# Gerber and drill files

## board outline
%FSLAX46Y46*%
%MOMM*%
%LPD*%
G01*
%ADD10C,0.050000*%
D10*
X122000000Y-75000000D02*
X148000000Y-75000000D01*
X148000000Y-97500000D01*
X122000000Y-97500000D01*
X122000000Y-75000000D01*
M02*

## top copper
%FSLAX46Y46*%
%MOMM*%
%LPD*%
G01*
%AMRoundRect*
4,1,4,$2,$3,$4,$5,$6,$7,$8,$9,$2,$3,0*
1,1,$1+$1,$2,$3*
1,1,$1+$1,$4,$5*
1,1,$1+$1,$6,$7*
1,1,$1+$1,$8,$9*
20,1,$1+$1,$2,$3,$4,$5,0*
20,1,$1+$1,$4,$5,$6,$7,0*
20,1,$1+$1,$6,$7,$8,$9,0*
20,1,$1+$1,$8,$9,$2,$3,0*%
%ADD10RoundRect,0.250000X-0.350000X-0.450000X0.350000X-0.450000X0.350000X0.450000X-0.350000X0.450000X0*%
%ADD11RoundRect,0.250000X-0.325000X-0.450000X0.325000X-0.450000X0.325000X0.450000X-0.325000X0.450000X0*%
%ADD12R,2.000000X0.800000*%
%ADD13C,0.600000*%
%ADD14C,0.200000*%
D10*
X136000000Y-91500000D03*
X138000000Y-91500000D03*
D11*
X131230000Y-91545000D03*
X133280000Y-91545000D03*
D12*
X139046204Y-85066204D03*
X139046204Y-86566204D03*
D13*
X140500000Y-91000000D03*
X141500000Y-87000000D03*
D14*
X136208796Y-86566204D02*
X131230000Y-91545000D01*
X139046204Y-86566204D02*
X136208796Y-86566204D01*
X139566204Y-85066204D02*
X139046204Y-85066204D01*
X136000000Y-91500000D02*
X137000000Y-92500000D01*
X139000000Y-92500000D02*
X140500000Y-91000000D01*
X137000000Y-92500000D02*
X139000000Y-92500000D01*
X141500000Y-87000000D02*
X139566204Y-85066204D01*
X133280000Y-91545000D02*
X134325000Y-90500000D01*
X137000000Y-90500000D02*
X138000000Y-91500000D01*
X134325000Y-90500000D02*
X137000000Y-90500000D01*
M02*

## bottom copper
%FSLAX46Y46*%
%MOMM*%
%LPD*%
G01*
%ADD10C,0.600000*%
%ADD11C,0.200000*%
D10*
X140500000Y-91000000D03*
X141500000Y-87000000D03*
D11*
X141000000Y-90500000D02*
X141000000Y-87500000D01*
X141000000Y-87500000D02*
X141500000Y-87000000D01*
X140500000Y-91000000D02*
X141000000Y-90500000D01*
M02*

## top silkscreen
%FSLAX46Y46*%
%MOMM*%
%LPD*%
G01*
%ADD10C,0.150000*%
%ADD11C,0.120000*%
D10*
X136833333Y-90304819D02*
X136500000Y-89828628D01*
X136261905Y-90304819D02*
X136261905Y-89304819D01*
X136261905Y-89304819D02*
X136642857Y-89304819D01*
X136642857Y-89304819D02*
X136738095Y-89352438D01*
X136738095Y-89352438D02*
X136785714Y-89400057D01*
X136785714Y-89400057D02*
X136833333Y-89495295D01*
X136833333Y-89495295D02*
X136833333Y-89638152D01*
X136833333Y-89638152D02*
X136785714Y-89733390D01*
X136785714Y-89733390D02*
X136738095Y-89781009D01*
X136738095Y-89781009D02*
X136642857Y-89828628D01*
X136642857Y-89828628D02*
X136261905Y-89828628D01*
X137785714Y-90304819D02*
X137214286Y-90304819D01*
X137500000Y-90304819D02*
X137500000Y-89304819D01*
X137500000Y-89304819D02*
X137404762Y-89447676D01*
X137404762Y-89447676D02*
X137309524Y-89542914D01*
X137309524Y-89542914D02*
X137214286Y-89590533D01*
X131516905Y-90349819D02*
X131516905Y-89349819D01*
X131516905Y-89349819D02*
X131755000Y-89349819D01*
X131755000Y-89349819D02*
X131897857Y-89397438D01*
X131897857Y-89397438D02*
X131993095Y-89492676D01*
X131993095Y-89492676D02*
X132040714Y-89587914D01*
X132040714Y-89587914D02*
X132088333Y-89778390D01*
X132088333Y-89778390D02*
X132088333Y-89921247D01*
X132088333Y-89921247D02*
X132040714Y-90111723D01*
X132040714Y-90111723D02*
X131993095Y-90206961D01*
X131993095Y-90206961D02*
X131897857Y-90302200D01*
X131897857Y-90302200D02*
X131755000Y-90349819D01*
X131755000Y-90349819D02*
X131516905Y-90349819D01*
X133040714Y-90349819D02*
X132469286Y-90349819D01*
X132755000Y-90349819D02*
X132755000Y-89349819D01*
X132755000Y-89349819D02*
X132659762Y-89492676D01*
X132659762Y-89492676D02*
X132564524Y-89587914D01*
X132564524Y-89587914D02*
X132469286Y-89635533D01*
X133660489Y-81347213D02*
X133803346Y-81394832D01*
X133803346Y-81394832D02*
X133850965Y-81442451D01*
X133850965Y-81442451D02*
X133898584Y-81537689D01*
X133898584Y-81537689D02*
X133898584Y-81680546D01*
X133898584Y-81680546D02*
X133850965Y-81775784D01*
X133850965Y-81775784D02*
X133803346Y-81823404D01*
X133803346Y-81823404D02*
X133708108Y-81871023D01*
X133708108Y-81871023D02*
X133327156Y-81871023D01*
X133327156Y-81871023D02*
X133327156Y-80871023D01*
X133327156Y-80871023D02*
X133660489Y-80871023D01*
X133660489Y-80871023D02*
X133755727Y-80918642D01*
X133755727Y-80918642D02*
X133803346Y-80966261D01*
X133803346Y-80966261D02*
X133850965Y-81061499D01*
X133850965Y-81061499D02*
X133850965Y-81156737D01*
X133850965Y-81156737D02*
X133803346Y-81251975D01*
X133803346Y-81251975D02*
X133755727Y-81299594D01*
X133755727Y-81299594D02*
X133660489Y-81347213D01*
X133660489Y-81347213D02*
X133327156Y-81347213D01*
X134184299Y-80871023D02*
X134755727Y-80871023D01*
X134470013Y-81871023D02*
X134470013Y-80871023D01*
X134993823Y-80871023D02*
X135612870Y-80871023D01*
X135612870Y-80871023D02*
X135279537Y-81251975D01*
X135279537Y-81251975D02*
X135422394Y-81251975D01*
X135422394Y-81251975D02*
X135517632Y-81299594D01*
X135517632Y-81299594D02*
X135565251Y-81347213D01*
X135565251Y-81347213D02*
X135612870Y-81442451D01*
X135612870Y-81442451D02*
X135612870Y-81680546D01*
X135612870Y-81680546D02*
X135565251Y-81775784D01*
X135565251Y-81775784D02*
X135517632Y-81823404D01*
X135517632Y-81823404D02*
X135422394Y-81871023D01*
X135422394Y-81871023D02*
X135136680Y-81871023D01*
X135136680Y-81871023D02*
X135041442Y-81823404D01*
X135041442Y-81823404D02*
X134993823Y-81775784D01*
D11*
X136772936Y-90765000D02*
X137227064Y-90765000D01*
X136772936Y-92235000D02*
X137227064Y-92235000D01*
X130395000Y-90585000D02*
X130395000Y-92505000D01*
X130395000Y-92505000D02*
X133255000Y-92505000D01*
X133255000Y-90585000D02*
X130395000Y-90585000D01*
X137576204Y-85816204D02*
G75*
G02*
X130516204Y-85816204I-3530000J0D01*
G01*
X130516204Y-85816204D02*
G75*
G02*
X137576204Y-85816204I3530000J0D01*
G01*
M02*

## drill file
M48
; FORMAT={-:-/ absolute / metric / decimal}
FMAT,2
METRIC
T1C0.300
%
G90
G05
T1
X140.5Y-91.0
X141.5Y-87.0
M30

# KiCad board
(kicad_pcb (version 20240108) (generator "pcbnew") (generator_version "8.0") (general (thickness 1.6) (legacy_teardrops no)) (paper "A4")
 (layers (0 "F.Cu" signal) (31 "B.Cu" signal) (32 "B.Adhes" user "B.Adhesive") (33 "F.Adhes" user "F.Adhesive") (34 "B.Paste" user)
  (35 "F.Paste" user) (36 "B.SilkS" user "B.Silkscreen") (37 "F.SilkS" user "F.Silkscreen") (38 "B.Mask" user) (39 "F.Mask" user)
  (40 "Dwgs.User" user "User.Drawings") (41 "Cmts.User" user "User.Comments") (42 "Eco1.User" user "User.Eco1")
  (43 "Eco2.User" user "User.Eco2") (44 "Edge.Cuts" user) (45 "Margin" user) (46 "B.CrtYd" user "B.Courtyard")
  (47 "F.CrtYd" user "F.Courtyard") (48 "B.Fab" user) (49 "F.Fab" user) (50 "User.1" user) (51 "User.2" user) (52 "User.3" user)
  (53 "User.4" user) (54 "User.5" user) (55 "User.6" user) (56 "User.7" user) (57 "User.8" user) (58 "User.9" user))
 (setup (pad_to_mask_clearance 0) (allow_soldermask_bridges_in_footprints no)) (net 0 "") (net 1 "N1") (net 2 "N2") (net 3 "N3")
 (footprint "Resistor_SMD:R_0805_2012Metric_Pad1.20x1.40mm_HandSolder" (layer "F.Cu") (at 137 91.5)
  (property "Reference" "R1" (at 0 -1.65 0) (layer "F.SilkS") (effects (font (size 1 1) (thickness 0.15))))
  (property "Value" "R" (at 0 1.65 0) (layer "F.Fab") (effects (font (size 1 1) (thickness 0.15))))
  (fp_line (start -0.227064 -0.735) (end 0.227064 -0.735) (stroke (width 0.12) (type solid)) (layer "F.SilkS"))
  (fp_line (start -0.227064 0.735) (end 0.227064 0.735) (stroke (width 0.12) (type solid)) (layer "F.SilkS"))
  (pad "1" smd roundrect (at -1 0) (size 1.2 1.4) (layers "F.Cu" "F.Paste" "F.Mask") (roundrect_rratio 0.208333) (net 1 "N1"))
  (pad "2" smd roundrect (at 1 0) (size 1.2 1.4) (layers "F.Cu" "F.Paste" "F.Mask") (roundrect_rratio 0.208333) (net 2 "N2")))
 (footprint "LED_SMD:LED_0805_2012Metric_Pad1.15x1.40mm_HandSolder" (layer "F.Cu") (at 132.255 91.545)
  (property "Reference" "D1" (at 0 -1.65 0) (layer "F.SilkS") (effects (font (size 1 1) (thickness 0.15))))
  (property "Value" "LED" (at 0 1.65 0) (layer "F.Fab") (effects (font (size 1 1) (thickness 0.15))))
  (fp_line (start -1.86 -0.96) (end -1.86 0.96) (stroke (width 0.12) (type solid)) (layer "F.SilkS"))
  (fp_line (start -1.86 0.96) (end 1 0.96) (stroke (width 0.12) (type solid)) (layer "F.SilkS"))
  (fp_line (start 1 -0.96) (end -1.86 -0.96) (stroke (width 0.12) (type solid)) (layer "F.SilkS"))
  (pad "1" smd roundrect (at -1.025 0) (size 1.15 1.4) (layers "F.Cu" "F.Paste" "F.Mask") (roundrect_rratio 0.217391) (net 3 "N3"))
  (pad "2" smd roundrect (at 1.025 0) (size 1.15 1.4) (layers "F.Cu" "F.Paste" "F.Mask") (roundrect_rratio 0.217391) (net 2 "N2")))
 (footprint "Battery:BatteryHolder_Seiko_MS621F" (layer "F.Cu") (at 139.046204 85.816204)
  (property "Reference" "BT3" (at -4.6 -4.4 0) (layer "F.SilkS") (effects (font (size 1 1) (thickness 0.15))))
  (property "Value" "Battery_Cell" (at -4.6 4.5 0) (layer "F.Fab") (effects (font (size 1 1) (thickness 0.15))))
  (fp_circle (center -5 0) (end -1.47 0) (stroke (width 0.12) (type solid)) (fill none) (layer "F.SilkS"))
  (pad "1" smd rect (at 0 -0.75) (size 2 0.8) (layers "F.Cu" "F.Paste" "F.Mask") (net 1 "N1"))
  (pad "2" smd rect (at 0 0.75) (size 2 0.8) (layers "F.Cu" "F.Paste" "F.Mask") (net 3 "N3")))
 (gr_rect (start 122 75) (end 148 97.5) (stroke (width 0.05) (type default)) (fill none) (layer "Edge.Cuts"))
 (segment (start 136.208796 86.566204) (end 131.23 91.545) (width 0.2) (layer "F.Cu") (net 3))
 (segment (start 139.046204 86.566204) (end 136.208796 86.566204) (width 0.2) (layer "F.Cu") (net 3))
 (segment (start 139.566204 85.066204) (end 139.046204 85.066204) (width 0.2) (layer "F.Cu") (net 1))
 (segment (start 136 91.5) (end 137 92.5) (width 0.2) (layer "F.Cu") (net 1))
 (segment (start 139 92.5) (end 140.5 91) (width 0.2) (layer "F.Cu") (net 1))
 (segment (start 137 92.5) (end 139 92.5) (width 0.2) (layer "F.Cu") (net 1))
 (segment (start 141.5 87) (end 139.566204 85.066204) (width 0.2) (layer "F.Cu") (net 1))
 (via (at 140.5 91) (size 0.6) (drill 0.3) (layers "F.Cu" "B.Cu") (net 1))
 (via (at 141.5 87) (size 0.6) (drill 0.3) (layers "F.Cu" "B.Cu") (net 1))
 (segment (start 141 90.5) (end 141 87.5) (width 0.2) (layer "B.Cu") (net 1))
 (segment (start 141 87.5) (end 141.5 87) (width 0.2) (layer "B.Cu") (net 1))
 (segment (start 140.5 91) (end 141 90.5) (width 0.2) (layer "B.Cu") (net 1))
 (segment (start 133.28 91.545) (end 134.325 90.5) (width 0.2) (layer "F.Cu") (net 2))
 (segment (start 137 90.5) (end 138 91.5) (width 0.2) (layer "F.Cu") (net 2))
 (segment (start 134.325 90.5) (end 137 90.5) (width 0.2) (layer "F.Cu") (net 2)))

